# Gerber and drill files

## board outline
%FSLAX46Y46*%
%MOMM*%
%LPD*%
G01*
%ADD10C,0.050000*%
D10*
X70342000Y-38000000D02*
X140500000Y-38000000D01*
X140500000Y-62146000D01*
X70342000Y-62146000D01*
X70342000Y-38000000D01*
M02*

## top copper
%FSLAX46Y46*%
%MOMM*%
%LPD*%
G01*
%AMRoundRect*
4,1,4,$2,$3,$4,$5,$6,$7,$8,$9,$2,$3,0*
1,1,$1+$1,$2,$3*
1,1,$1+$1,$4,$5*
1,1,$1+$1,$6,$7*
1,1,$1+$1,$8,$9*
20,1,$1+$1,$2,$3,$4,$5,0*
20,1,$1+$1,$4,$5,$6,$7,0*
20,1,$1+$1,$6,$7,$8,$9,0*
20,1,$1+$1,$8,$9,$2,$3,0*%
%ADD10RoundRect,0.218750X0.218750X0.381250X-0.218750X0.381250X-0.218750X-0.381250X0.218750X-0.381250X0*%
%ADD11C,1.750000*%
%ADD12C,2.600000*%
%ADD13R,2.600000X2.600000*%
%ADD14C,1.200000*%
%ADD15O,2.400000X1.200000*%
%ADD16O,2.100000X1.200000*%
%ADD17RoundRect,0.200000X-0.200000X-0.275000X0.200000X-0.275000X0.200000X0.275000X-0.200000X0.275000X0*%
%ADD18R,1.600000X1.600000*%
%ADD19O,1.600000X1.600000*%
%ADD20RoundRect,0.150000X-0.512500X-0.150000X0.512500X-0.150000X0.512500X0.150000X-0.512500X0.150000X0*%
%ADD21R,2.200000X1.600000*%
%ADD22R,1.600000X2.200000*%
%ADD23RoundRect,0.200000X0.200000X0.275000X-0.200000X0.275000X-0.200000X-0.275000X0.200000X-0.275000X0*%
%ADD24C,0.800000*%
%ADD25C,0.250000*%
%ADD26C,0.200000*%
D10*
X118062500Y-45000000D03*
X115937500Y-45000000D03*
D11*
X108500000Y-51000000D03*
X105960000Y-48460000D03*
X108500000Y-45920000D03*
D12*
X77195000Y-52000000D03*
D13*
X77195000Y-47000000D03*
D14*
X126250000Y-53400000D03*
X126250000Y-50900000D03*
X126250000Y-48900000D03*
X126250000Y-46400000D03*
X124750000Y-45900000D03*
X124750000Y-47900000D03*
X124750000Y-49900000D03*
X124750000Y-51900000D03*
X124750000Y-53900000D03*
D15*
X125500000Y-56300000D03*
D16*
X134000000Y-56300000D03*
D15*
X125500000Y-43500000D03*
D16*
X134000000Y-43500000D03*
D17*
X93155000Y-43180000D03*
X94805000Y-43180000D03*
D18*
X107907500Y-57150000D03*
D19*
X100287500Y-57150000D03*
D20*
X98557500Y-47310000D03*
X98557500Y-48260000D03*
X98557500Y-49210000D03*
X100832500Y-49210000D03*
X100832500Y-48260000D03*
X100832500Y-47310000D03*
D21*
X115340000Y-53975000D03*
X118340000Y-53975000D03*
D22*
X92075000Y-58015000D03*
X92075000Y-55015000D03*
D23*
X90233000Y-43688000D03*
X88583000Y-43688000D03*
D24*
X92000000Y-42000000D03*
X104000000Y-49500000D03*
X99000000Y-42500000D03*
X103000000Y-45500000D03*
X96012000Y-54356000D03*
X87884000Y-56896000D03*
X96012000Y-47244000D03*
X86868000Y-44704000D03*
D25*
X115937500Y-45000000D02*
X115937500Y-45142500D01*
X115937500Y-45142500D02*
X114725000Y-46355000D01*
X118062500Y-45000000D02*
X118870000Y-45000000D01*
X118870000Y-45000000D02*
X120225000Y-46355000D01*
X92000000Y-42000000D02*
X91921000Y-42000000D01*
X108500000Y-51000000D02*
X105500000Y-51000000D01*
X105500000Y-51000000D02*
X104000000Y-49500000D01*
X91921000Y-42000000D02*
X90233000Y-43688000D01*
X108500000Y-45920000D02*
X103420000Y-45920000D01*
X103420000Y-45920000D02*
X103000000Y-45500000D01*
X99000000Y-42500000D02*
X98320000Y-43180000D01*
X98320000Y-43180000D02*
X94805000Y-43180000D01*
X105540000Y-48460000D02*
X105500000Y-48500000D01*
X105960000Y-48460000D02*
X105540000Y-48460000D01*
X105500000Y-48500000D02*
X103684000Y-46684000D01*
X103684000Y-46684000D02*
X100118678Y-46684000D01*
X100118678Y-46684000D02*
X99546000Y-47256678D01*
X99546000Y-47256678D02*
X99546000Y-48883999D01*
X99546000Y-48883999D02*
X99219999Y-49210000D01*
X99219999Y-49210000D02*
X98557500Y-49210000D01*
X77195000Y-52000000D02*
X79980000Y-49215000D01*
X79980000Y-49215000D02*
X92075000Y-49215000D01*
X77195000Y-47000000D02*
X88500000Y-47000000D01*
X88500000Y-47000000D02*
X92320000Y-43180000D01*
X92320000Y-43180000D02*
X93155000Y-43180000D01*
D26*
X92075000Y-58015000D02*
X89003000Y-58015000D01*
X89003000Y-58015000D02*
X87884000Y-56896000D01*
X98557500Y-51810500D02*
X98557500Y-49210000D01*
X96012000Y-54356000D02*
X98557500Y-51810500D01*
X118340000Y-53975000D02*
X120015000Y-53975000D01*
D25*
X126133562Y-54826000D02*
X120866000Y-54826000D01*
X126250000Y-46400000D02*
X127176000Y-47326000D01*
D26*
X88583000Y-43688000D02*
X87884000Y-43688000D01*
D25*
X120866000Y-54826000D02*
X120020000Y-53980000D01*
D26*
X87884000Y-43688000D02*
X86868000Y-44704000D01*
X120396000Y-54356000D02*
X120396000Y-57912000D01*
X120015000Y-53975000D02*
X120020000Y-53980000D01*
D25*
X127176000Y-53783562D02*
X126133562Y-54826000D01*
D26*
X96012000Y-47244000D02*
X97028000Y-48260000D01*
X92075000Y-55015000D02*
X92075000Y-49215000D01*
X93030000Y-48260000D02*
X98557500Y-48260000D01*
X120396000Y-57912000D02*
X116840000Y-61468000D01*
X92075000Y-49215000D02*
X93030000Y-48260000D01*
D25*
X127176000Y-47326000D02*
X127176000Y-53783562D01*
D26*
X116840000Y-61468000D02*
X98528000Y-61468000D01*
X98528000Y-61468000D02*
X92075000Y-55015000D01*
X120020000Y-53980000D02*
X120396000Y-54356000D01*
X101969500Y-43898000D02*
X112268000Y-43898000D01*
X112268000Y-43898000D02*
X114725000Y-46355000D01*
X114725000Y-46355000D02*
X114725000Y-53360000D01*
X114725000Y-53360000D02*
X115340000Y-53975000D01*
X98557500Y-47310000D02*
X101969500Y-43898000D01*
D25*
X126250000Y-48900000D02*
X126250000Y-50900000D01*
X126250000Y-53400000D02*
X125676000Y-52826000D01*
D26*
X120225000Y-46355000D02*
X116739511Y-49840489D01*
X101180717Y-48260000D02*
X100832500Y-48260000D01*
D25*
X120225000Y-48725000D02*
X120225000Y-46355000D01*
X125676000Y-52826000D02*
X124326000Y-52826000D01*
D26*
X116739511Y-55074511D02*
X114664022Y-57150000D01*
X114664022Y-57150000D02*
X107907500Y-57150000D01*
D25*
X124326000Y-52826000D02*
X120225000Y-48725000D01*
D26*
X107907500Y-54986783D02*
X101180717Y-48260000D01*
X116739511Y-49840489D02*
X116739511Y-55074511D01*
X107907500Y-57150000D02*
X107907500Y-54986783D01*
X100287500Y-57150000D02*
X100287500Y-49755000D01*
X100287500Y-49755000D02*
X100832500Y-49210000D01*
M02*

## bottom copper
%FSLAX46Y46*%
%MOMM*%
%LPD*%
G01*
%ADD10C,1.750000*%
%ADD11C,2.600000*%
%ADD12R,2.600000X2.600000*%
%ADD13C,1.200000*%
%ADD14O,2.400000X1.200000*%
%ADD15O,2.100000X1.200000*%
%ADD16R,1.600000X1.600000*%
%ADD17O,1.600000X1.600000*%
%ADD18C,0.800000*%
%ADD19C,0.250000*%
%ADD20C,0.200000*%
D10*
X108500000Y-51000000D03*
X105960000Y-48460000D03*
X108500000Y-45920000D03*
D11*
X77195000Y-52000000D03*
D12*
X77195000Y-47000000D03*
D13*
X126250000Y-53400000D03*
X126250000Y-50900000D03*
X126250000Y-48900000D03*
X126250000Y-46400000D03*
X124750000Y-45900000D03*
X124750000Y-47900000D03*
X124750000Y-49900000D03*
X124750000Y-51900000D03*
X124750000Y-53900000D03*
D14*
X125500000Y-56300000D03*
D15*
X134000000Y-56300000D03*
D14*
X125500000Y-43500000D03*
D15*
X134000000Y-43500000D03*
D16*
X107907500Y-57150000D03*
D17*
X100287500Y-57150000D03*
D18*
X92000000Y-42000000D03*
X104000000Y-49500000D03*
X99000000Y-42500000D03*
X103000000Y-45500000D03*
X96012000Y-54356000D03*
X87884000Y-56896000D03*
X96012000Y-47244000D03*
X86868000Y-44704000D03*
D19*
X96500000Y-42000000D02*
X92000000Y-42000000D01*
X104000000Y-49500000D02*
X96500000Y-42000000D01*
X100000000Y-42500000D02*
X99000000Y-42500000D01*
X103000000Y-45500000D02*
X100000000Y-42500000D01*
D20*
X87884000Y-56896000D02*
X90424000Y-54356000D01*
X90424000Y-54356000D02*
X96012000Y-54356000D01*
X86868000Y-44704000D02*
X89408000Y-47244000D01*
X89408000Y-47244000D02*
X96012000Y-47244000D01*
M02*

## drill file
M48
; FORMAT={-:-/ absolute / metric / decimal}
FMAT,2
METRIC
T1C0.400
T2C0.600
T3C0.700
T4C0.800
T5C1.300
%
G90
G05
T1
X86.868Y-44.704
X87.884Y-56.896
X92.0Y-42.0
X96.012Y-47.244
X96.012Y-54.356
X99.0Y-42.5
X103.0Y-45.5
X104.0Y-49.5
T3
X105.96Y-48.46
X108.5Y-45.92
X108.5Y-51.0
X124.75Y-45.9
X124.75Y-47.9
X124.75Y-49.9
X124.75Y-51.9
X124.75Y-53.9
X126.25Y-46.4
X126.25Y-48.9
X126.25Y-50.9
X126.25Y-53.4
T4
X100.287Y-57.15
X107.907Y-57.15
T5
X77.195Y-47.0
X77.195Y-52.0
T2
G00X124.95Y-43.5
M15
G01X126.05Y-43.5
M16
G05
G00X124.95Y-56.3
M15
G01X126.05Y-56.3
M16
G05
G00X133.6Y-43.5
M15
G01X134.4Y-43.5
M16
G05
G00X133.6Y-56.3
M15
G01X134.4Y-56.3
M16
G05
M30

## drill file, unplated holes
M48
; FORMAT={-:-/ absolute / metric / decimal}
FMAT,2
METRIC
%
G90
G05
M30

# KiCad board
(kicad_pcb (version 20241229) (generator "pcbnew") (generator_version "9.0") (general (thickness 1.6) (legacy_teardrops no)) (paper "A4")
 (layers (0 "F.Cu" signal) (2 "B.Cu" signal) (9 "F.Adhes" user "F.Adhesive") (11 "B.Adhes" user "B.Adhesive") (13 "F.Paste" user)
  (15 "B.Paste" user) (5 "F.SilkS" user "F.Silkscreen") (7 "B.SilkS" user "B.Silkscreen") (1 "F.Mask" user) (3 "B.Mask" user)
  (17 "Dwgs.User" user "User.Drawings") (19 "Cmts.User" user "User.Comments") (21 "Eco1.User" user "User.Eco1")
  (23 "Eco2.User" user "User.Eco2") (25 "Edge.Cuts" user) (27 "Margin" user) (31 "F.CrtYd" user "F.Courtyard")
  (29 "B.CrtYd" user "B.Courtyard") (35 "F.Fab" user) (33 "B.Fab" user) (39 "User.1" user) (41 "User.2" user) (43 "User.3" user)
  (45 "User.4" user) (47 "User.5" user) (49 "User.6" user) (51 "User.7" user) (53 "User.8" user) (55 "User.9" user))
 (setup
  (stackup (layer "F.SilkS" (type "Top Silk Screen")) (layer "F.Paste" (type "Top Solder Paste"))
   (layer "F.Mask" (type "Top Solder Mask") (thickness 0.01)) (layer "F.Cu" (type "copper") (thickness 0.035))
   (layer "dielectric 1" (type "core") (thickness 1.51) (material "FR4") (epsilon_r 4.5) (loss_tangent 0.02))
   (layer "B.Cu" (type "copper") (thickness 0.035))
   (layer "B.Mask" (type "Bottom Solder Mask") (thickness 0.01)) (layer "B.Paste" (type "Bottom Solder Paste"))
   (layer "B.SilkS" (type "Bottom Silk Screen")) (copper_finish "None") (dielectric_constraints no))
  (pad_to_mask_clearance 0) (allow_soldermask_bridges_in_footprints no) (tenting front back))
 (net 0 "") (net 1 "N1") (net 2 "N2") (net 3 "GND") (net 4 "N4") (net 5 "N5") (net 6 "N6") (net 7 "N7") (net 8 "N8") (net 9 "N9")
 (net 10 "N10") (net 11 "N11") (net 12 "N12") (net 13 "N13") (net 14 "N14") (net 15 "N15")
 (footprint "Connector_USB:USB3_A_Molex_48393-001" (layer "F.Cu") (at 126.25 53.4 90)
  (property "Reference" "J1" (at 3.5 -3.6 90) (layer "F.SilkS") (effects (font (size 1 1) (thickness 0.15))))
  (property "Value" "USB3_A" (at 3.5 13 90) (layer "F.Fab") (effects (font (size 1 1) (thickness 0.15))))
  (pad "1" thru_hole circle (at 0 0 90) (size 1.2 1.2) (drill 0.7) (layers "*.Cu" "*.Mask") (remove_unused_layers no) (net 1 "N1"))
  (pad "2" thru_hole circle (at 2.5 0 90) (size 1.2 1.2) (drill 0.7) (layers "*.Cu" "*.Mask") (remove_unused_layers no) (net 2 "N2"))
  (pad "3" thru_hole circle (at 4.5 0 90) (size 1.2 1.2) (drill 0.7) (layers "*.Cu" "*.Mask") (remove_unused_layers no) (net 2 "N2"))
  (pad "4" thru_hole circle (at 7 0 90) (size 1.2 1.2) (drill 0.7) (layers "*.Cu" "*.Mask") (remove_unused_layers no) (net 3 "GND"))
  (pad "5" thru_hole circle (at 7.5 -1.5 90) (size 1.2 1.2) (drill 0.7) (layers "*.Cu" "*.Mask") (remove_unused_layers no) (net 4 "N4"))
  (pad "6" thru_hole circle (at 5.5 -1.5 90) (size 1.2 1.2) (drill 0.7) (layers "*.Cu" "*.Mask") (remove_unused_layers no) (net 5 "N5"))
  (pad "7" thru_hole circle (at 3.5 -1.5 90) (size 1.2 1.2) (drill 0.7) (layers "*.Cu" "*.Mask") (remove_unused_layers no) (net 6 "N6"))
  (pad "8" thru_hole circle (at 1.5 -1.5 90) (size 1.2 1.2) (drill 0.7) (layers "*.Cu" "*.Mask") (remove_unused_layers no) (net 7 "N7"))
  (pad "9" thru_hole circle (at -0.5 -1.5 90) (size 1.2 1.2) (drill 0.7) (layers "*.Cu" "*.Mask") (remove_unused_layers no) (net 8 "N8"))
  (pad "10" thru_hole oval (at -2.9 -0.75 90) (size 1.2 2.4) (drill oval 0.6 1.7) (layers "*.Cu" "*.Mask") (remove_unused_layers no)
   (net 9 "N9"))
  (pad "10" thru_hole oval (at -2.9 7.75 90) (size 1.2 2.1) (drill oval 0.6 1.4) (layers "*.Cu" "*.Mask") (remove_unused_layers no)
   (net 9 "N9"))
  (pad "10" thru_hole oval (at 9.9 -0.75 90) (size 1.2 2.4) (drill oval 0.6 1.7) (layers "*.Cu" "*.Mask") (remove_unused_layers no)
   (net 9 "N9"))
  (pad "10" thru_hole oval (at 9.9 7.75 90) (size 1.2 2.1) (drill oval 0.6 1.4) (layers "*.Cu" "*.Mask") (remove_unused_layers no)
   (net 9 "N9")))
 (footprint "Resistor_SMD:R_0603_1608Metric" (layer "F.Cu") (at 93.98 43.18)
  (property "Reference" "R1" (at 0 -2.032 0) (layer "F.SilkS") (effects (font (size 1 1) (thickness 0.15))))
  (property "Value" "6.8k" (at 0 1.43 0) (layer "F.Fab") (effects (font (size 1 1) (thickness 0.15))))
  (pad "1" smd roundrect (at -0.825 0) (size 0.8 0.95) (layers "F.Cu" "F.Mask" "F.Paste") (roundrect_rratio 0.25) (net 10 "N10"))
  (pad "2" smd roundrect (at 0.825 0) (size 0.8 0.95) (layers "F.Cu" "F.Mask" "F.Paste") (roundrect_rratio 0.25) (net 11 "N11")))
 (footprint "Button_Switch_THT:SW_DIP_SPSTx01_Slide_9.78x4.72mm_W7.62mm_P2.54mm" (layer "F.Cu") (at 107.9075 57.15 180)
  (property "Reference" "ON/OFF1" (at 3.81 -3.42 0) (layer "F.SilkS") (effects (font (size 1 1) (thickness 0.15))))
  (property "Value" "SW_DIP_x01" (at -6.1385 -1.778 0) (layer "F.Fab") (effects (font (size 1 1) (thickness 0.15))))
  (pad "1" thru_hole rect (at 0 0 180) (size 1.6 1.6) (drill 0.8) (layers "*.Cu" "*.Mask") (remove_unused_layers no) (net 1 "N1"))
  (pad "2" thru_hole oval (at 7.62 0 180) (size 1.6 1.6) (drill 0.8) (layers "*.Cu" "*.Mask") (remove_unused_layers no) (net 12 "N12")))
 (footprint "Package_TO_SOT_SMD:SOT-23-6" (layer "F.Cu") (at 99.695 48.26)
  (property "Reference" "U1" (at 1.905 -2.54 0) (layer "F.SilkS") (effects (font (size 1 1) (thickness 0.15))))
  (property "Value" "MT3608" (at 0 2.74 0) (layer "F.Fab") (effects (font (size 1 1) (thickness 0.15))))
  (pad "1" smd roundrect (at -1.1375 -0.95) (size 1.325 0.6) (layers "F.Cu" "F.Mask" "F.Paste") (roundrect_rratio 0.25) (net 10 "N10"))
  (pad "2" smd roundrect (at -1.1375 0) (size 1.325 0.6) (layers "F.Cu" "F.Mask" "F.Paste") (roundrect_rratio 0.25) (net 3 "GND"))
  (pad "3" smd roundrect (at -1.1375 0.95) (size 1.325 0.6) (layers "F.Cu" "F.Mask" "F.Paste") (roundrect_rratio 0.25) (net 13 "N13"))
  (pad "4" smd roundrect (at 1.1375 0.95) (size 1.325 0.6) (layers "F.Cu" "F.Mask" "F.Paste") (roundrect_rratio 0.25) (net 12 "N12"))
  (pad "5" smd roundrect (at 1.1375 0) (size 1.325 0.6) (layers "F.Cu" "F.Mask" "F.Paste") (roundrect_rratio 0.25) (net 1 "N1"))
  (pad "6" smd roundrect (at 1.1375 -0.95) (size 1.325 0.6) (layers "F.Cu" "F.Mask" "F.Paste") (roundrect_rratio 0.25) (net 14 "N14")))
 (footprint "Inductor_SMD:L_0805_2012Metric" (layer "F.Cu") (at 117 45 180)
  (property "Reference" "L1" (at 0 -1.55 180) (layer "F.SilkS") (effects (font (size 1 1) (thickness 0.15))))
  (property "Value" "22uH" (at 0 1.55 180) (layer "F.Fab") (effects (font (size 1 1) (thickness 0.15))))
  (pad "1" smd roundrect (at -1.0625 0 180) (size 0.875 1.2) (layers "F.Cu" "F.Mask" "F.Paste") (roundrect_rratio 0.25) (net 1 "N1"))
  (pad "2" smd roundrect (at 1.0625 0 180) (size 0.875 1.2) (layers "F.Cu" "F.Mask" "F.Paste") (roundrect_rratio 0.25) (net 10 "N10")))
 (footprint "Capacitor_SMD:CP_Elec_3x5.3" (layer "F.Cu") (at 116.84 53.975)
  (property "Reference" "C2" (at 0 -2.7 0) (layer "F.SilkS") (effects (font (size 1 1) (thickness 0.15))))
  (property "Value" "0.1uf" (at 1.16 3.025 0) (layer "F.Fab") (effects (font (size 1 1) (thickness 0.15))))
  (pad "1" smd rect (at -1.5 0) (size 2.2 1.6) (layers "F.Cu" "F.Mask" "F.Paste") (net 10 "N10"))
  (pad "2" smd rect (at 1.5 0) (size 2.2 1.6) (layers "F.Cu" "F.Mask" "F.Paste") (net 3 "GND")))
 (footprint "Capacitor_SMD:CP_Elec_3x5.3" (layer "F.Cu") (at 92.075 56.515 90)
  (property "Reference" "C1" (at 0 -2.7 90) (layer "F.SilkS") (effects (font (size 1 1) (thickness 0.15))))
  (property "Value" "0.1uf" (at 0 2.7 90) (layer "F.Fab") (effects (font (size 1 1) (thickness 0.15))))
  (pad "1" smd rect (at -1.5 0 90) (size 2.2 1.6) (layers "F.Cu" "F.Mask" "F.Paste") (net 13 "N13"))
  (pad "2" smd rect (at 1.5 0 90) (size 2.2 1.6) (layers "F.Cu" "F.Mask" "F.Paste") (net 3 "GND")))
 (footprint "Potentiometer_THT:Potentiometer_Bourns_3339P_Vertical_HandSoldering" (layer "F.Cu") (at 108.5 51)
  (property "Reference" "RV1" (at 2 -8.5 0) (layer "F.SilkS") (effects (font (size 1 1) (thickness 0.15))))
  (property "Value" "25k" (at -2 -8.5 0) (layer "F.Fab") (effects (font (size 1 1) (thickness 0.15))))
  (pad "1" thru_hole circle (at 0 0) (size 1.75 1.75) (drill 0.7) (layers "*.Cu" "*.Mask") (remove_unused_layers no) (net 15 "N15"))
  (pad "2" thru_hole circle (at -2.54 -2.54) (size 1.75 1.75) (drill 0.7) (layers "*.Cu" "*.Mask") (remove_unused_layers no) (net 13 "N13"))
  (pad "3" thru_hole circle (at 0 -5.08) (size 1.75 1.75) (drill 0.7) (layers "*.Cu" "*.Mask") (remove_unused_layers no) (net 11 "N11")))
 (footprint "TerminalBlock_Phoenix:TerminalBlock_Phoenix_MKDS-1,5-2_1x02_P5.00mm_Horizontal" (layer "F.Cu") (at 77.195 47 -90)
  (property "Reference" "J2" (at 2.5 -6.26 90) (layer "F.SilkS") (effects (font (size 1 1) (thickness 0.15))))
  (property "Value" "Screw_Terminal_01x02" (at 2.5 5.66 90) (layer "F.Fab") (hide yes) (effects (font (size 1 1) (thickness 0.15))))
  (pad "1" thru_hole rect (at 0 0 270) (size 2.6 2.6) (drill 1.3) (layers "*.Cu" "*.Mask") (remove_unused_layers no) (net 10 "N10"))
  (pad "2" thru_hole circle (at 5 0 270) (size 2.6 2.6) (drill 1.3) (layers "*.Cu" "*.Mask") (remove_unused_layers no) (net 3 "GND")))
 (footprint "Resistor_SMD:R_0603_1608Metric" (layer "F.Cu") (at 89.408 43.688 180)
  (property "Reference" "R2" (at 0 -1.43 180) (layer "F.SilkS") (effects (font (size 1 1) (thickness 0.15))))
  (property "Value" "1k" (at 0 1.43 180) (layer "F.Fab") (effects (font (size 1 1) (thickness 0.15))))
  (pad "1" smd roundrect (at -0.825 0 180) (size 0.8 0.95) (layers "F.Cu" "F.Mask" "F.Paste") (roundrect_rratio 0.25) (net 15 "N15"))
  (pad "2" smd roundrect (at 0.825 0 180) (size 0.8 0.95) (layers "F.Cu" "F.Mask" "F.Paste") (roundrect_rratio 0.25) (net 3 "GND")))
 (gr_rect (start 70.342 38) (end 140.5 62.146) (stroke (width 0.05) (type solid)) (fill no) (layer "Edge.Cuts"))
 (segment (start 105.54 48.46) (end 105.5 48.5) (width 0.25) (layer "F.Cu") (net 13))
 (segment (start 92.075 58.015) (end 89.003 58.015) (width 0.2) (layer "F.Cu") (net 13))
 (segment (start 89.003 58.015) (end 87.884 56.896) (width 0.2) (layer "F.Cu") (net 13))
 (segment (start 98.5575 51.8105) (end 98.5575 49.21) (width 0.2) (layer "F.Cu") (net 13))
 (segment (start 99.546 48.883999) (end 99.219999 49.21) (width 0.25) (layer "F.Cu") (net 13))
 (segment (start 100.118678 46.684) (end 99.546 47.256678) (width 0.25) (layer "F.Cu") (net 13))
 (segment (start 105.5 48.5) (end 103.684 46.684) (width 0.25) (layer "F.Cu") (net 13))
 (segment (start 99.546 47.256678) (end 99.546 48.883999) (width 0.25) (layer "F.Cu") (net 13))
 (segment (start 103.684 46.684) (end 100.118678 46.684) (width 0.25) (layer "F.Cu") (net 13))
 (segment (start 105.96 48.46) (end 105.54 48.46) (width 0.25) (layer "F.Cu") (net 13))
 (segment (start 99.219999 49.21) (end 98.5575 49.21) (width 0.25) (layer "F.Cu") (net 13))
 (segment (start 96.012 54.356) (end 98.5575 51.8105) (width 0.2) (layer "F.Cu") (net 13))
 (via (at 96.012 54.356) (size 0.8) (drill 0.4) (layers "F.Cu" "B.Cu") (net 13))
 (via (at 87.884 56.896) (size 0.8) (drill 0.4) (layers "F.Cu" "B.Cu") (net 13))
 (segment (start 87.884 56.896) (end 90.424 54.356) (width 0.2) (layer "B.Cu") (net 13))
 (segment (start 90.424 54.356) (end 96.012 54.356) (width 0.2) (layer "B.Cu") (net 13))
 (segment (start 118.34 53.975) (end 120.015 53.975) (width 0.2) (layer "F.Cu") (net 3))
 (segment (start 126.133562 54.826) (end 120.866 54.826) (width 0.25) (layer "F.Cu") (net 3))
 (segment (start 126.25 46.4) (end 127.176 47.326) (width 0.25) (layer "F.Cu") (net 3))
 (segment (start 88.583 43.688) (end 87.884 43.688) (width 0.2) (layer "F.Cu") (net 3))
 (segment (start 120.866 54.826) (end 120.02 53.98) (width 0.25) (layer "F.Cu") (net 3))
 (segment (start 87.884 43.688) (end 86.868 44.704) (width 0.2) (layer "F.Cu") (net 3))
 (segment (start 120.396 54.356) (end 120.396 57.912) (width 0.2) (layer "F.Cu") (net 3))
 (segment (start 120.015 53.975) (end 120.02 53.98) (width 0.2) (layer "F.Cu") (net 3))
 (segment (start 127.176 53.783562) (end 126.133562 54.826) (width 0.25) (layer "F.Cu") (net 3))
 (segment (start 96.012 47.244) (end 97.028 48.26) (width 0.2) (layer "F.Cu") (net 3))
 (segment (start 92.075 55.015) (end 92.075 49.215) (width 0.2) (layer "F.Cu") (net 3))
 (segment (start 93.03 48.26) (end 98.5575 48.26) (width 0.2) (layer "F.Cu") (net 3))
 (segment (start 77.195 52) (end 79.98 49.215) (width 0.25) (layer "F.Cu") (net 3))
 (segment (start 120.396 57.912) (end 116.84 61.468) (width 0.2) (layer "F.Cu") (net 3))
 (segment (start 92.075 49.215) (end 93.03 48.26) (width 0.2) (layer "F.Cu") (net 3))
 (segment (start 127.176 47.326) (end 127.176 53.783562) (width 0.25) (layer "F.Cu") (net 3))
 (segment (start 116.84 61.468) (end 98.528 61.468) (width 0.2) (layer "F.Cu") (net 3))
 (segment (start 79.98 49.215) (end 92.075 49.215) (width 0.25) (layer "F.Cu") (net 3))
 (segment (start 98.528 61.468) (end 92.075 55.015) (width 0.2) (layer "F.Cu") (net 3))
 (segment (start 120.02 53.98) (end 120.396 54.356) (width 0.2) (layer "F.Cu") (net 3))
 (via (at 96.012 47.244) (size 0.8) (drill 0.4) (layers "F.Cu" "B.Cu") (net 3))
 (via (at 86.868 44.704) (size 0.8) (drill 0.4) (layers "F.Cu" "B.Cu") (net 3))
 (segment (start 86.868 44.704) (end 89.408 47.244) (width 0.2) (layer "B.Cu") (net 3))
 (segment (start 89.408 47.244) (end 96.012 47.244) (width 0.2) (layer "B.Cu") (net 3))
 (segment (start 88.5 47) (end 92.32 43.18) (width 0.25) (layer "F.Cu") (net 10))
 (segment (start 101.9695 43.898) (end 112.268 43.898) (width 0.2) (layer "F.Cu") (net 10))
 (segment (start 92.32 43.18) (end 93.155 43.18) (width 0.25) (layer "F.Cu") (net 10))
 (segment (start 112.268 43.898) (end 114.725 46.355) (width 0.2) (layer "F.Cu") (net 10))
 (segment (start 115.9375 45.1425) (end 114.725 46.355) (width 0.25) (layer "F.Cu") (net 10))
 (segment (start 114.725 46.355) (end 114.725 53.36) (width 0.2) (layer "F.Cu") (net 10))
 (segment (start 77.195 47) (end 88.5 47) (width 0.25) (layer "F.Cu") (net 10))
 (segment (start 114.725 53.36) (end 115.34 53.975) (width 0.2) (layer "F.Cu") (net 10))
 (segment (start 98.5575 47.31) (end 101.9695 43.898) (width 0.2) (layer "F.Cu") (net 10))
 (segment (start 115.9375 45) (end 115.9375 45.1425) (width 0.25) (layer "F.Cu") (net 10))
 (segment (start 126.25 48.9) (end 126.25 50.9) (width 0.25) (layer "F.Cu") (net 2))
 (segment (start 118.87 45) (end 120.225 46.355) (width 0.25) (layer "F.Cu") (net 1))
 (segment (start 126.25 53.4) (end 125.676 52.826) (width 0.25) (layer "F.Cu") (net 1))
 (segment (start 120.225 46.355) (end 116.739511 49.840489) (width 0.2) (layer "F.Cu") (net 1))
 (segment (start 101.180717 48.26) (end 100.8325 48.26) (width 0.2) (layer "F.Cu") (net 1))
 (segment (start 120.225 48.725) (end 120.225 46.355) (width 0.25) (layer "F.Cu") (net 1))
 (segment (start 125.676 52.826) (end 124.326 52.826) (width 0.25) (layer "F.Cu") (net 1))
 (segment (start 116.739511 55.074511) (end 114.664022 57.15) (width 0.2) (layer "F.Cu") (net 1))
 (segment (start 114.664022 57.15) (end 107.9075 57.15) (width 0.2) (layer "F.Cu") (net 1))
 (segment (start 124.326 52.826) (end 120.225 48.725) (width 0.25) (layer "F.Cu") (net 1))
 (segment (start 107.9075 54.986783) (end 101.180717 48.26) (width 0.2) (layer "F.Cu") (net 1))
 (segment (start 116.739511 49.840489) (end 116.739511 55.074511) (width 0.2) (layer "F.Cu") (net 1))
 (segment (start 107.9075 57.15) (end 107.9075 54.986783) (width 0.2) (layer "F.Cu") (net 1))
 (segment (start 118.0625 45) (end 118.87 45) (width 0.25) (layer "F.Cu") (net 1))
 (segment (start 100.2875 57.15) (end 100.2875 49.755) (width 0.2) (layer "F.Cu") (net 12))
 (segment (start 100.2875 49.755) (end 100.8325 49.21) (width 0.2) (layer "F.Cu") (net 12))
 (segment (start 103.42 45.92) (end 103 45.5) (width 0.25) (layer "F.Cu") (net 11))
 (segment (start 99 42.5) (end 98.32 43.18) (width 0.25) (layer "F.Cu") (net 11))
 (segment (start 108.5 45.92) (end 103.42 45.92) (width 0.25) (layer "F.Cu") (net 11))
 (segment (start 98.32 43.18) (end 94.805 43.18) (width 0.25) (layer "F.Cu") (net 11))
 (via (at 103 45.5) (size 0.8) (drill 0.4) (layers "F.Cu" "B.Cu") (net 11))
 (via (at 99 42.5) (size 0.8) (drill 0.4) (layers "F.Cu" "B.Cu") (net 11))
 (segment (start 100 42.5) (end 99 42.5) (width 0.25) (layer "B.Cu") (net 11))
 (segment (start 103 45.5) (end 100 42.5) (width 0.25) (layer "B.Cu") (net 11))
 (segment (start 108.5 51) (end 105.5 51) (width 0.25) (layer "F.Cu") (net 15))
 (segment (start 105.5 51) (end 104 49.5) (width 0.25) (layer "F.Cu") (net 15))
 (segment (start 92 42) (end 91.921 42) (width 0.25) (layer "F.Cu") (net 15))
 (segment (start 91.921 42) (end 90.233 43.688) (width 0.25) (layer "F.Cu") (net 15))
 (via (at 92 42) (size 0.8) (drill 0.4) (layers "F.Cu" "B.Cu") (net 15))
 (via (at 104 49.5) (size 0.8) (drill 0.4) (layers "F.Cu" "B.Cu") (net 15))
 (segment (start 104 49.5) (end 96.5 42) (width 0.25) (layer "B.Cu") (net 15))
 (segment (start 96.5 42) (end 92 42) (width 0.25) (layer "B.Cu") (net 15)))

